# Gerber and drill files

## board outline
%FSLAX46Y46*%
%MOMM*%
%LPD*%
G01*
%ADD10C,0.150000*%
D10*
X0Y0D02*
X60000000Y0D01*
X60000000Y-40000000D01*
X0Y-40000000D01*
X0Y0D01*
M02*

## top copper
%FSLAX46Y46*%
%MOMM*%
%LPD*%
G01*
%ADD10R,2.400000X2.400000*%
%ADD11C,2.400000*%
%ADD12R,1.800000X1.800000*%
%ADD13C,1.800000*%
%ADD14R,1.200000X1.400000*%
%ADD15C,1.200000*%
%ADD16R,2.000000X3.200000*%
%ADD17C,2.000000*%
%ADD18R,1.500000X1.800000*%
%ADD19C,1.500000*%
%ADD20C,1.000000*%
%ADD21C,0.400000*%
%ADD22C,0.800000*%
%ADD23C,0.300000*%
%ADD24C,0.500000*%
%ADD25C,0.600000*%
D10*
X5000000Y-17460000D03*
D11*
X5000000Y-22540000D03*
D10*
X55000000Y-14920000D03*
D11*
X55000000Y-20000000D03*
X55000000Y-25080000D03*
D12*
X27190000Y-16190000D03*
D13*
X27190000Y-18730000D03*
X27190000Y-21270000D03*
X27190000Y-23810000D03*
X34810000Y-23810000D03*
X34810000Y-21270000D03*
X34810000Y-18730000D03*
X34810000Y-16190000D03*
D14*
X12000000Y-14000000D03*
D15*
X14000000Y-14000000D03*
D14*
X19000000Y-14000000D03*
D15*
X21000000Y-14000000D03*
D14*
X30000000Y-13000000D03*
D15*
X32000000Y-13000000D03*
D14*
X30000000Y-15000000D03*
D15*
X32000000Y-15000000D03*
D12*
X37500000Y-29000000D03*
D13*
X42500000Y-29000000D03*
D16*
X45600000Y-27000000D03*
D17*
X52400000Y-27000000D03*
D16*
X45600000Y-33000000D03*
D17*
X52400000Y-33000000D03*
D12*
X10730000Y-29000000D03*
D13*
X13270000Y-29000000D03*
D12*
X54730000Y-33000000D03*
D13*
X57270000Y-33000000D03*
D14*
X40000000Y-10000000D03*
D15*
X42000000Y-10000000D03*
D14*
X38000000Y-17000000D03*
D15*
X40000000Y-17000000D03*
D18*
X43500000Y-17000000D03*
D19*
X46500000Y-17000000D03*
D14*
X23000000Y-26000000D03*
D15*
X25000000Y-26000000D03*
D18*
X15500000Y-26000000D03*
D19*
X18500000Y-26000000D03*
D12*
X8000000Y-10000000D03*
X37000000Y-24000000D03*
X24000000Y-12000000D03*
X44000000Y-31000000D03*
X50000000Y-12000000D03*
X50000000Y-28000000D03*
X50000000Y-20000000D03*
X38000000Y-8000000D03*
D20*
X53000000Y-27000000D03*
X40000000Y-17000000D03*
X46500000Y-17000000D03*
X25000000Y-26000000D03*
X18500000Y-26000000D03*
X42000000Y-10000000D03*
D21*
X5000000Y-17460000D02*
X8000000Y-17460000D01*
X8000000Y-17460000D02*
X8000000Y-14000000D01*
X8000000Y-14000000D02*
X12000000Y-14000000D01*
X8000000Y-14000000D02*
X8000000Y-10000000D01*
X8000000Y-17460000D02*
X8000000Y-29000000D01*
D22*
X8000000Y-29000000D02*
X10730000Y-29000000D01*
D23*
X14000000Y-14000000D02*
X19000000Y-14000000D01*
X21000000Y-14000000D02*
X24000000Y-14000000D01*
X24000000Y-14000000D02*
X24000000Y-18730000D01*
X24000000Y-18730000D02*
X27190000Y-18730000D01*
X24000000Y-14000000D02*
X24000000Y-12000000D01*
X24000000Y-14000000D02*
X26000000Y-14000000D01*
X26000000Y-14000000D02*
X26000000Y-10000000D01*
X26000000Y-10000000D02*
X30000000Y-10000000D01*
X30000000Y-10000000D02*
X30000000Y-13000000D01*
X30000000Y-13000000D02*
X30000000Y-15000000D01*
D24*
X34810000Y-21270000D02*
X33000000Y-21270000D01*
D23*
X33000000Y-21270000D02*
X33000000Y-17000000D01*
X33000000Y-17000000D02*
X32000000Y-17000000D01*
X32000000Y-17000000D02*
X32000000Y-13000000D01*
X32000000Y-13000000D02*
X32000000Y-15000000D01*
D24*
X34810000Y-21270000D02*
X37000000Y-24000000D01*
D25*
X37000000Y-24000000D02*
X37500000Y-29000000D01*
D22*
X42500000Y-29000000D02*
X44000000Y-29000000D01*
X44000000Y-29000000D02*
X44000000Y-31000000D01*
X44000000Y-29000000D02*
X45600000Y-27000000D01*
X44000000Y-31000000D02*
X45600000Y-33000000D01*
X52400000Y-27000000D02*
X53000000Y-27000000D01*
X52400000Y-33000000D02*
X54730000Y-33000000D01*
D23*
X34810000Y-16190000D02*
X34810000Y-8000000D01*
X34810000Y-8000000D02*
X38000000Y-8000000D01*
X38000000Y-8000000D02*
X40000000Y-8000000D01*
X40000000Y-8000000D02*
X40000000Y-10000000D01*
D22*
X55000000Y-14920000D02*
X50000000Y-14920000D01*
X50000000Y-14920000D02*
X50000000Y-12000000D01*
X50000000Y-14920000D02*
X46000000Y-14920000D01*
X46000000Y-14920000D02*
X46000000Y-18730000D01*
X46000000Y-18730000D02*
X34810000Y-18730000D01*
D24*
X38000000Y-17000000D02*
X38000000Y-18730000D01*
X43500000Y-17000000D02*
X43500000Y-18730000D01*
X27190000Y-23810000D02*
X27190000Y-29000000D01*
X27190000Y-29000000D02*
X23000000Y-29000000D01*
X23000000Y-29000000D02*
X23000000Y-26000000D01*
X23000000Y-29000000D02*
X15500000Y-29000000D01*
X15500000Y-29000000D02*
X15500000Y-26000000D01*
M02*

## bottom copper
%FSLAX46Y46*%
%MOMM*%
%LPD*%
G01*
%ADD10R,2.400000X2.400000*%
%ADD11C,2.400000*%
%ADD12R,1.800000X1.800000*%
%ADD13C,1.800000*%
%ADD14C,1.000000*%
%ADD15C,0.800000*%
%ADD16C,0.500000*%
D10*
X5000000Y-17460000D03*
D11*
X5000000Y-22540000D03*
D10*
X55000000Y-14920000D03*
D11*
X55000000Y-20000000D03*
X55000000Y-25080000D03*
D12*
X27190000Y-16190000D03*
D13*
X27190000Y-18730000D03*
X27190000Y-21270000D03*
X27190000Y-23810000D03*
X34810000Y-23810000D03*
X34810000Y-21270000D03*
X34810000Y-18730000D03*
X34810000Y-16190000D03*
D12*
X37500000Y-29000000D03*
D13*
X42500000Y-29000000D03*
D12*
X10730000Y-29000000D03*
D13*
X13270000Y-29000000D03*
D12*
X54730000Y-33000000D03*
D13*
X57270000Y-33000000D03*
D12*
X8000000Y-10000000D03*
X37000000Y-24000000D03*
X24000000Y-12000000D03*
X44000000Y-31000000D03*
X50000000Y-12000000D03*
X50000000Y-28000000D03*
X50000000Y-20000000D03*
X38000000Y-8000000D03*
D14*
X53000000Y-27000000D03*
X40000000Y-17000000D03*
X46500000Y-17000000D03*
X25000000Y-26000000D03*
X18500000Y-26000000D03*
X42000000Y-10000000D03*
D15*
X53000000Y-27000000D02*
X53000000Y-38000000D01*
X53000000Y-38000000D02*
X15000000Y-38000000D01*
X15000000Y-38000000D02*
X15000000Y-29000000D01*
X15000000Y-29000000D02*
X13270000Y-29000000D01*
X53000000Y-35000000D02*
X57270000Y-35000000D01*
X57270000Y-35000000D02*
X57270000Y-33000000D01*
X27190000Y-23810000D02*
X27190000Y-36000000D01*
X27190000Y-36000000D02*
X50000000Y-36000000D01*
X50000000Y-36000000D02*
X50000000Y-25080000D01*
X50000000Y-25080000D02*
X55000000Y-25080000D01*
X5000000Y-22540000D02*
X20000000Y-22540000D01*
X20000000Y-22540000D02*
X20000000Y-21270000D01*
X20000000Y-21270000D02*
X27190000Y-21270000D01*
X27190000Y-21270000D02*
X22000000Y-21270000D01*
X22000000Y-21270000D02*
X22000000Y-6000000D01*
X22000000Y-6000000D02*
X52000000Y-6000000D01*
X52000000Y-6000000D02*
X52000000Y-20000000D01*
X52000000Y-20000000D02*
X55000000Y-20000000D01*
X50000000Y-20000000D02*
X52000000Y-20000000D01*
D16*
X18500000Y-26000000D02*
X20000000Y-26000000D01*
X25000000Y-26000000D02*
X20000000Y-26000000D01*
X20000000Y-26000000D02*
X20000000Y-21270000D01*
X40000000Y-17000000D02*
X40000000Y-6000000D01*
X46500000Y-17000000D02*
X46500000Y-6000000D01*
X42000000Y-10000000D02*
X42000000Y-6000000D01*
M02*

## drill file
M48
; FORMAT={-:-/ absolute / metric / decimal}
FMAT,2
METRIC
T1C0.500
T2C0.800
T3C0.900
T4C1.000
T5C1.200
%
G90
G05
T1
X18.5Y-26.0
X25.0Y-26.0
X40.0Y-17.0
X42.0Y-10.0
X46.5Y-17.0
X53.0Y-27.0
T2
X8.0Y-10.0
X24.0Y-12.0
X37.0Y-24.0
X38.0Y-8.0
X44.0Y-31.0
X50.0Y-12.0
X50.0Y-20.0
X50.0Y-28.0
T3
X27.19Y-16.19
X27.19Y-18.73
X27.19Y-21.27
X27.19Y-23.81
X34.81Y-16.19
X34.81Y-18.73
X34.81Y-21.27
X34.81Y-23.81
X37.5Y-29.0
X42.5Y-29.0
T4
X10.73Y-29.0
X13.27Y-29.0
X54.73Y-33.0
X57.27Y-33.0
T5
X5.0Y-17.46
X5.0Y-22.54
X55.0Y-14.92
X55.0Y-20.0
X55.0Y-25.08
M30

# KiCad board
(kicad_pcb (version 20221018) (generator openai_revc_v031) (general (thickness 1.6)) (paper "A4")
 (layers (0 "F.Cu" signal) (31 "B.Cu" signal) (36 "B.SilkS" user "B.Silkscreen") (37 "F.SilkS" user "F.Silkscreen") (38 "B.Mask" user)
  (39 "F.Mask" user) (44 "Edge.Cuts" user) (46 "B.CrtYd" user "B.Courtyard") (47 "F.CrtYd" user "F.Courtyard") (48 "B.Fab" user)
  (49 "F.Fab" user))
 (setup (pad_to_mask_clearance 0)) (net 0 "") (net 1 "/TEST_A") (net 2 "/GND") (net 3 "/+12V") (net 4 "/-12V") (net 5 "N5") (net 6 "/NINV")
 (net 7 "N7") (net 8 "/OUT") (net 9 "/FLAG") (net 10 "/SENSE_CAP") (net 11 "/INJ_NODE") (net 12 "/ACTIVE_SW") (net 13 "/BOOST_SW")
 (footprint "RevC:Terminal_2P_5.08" (layer "F.Cu") (at 5.00 20.00)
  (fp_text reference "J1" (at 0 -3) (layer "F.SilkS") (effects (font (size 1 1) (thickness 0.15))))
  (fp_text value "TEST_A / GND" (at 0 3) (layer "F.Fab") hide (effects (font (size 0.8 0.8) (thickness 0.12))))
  (pad "1" thru_hole rect (at 0.00 -2.54) (size 2.40 2.40) (drill 1.20) (layers "*.Cu" "*.Mask") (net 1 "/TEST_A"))
  (pad "2" thru_hole circle (at 0.00 2.54) (size 2.40 2.40) (drill 1.20) (layers "*.Cu" "*.Mask") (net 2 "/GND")))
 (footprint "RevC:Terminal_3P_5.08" (layer "F.Cu") (at 55.00 20.00)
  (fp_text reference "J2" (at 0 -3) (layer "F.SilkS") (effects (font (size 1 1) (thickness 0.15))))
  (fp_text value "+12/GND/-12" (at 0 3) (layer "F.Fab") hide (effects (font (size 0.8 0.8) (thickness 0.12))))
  (pad "1" thru_hole rect (at 0.00 -5.08) (size 2.40 2.40) (drill 1.20) (layers "*.Cu" "*.Mask") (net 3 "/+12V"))
  (pad "2" thru_hole circle (at 0.00 0.00) (size 2.40 2.40) (drill 1.20) (layers "*.Cu" "*.Mask") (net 2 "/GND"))
  (pad "3" thru_hole circle (at 0.00 5.08) (size 2.40 2.40) (drill 1.20) (layers "*.Cu" "*.Mask") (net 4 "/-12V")))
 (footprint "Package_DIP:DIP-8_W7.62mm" (layer "F.Cu") (at 31.00 20.00)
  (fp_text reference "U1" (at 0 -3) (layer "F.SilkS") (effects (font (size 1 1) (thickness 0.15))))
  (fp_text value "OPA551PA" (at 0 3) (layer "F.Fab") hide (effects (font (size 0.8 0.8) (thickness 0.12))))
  (pad "1" thru_hole rect (at -3.81 -3.81) (size 1.80 1.80) (drill 0.90) (layers "*.Cu" "*.Mask") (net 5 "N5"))
  (pad "2" thru_hole circle (at -3.81 -1.27) (size 1.80 1.80) (drill 0.90) (layers "*.Cu" "*.Mask") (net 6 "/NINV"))
  (pad "3" thru_hole circle (at -3.81 1.27) (size 1.80 1.80) (drill 0.90) (layers "*.Cu" "*.Mask") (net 2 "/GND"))
  (pad "4" thru_hole circle (at -3.81 3.81) (size 1.80 1.80) (drill 0.90) (layers "*.Cu" "*.Mask") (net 4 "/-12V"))
  (pad "5" thru_hole circle (at 3.81 3.81) (size 1.80 1.80) (drill 0.90) (layers "*.Cu" "*.Mask") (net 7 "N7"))
  (pad "6" thru_hole circle (at 3.81 1.27) (size 1.80 1.80) (drill 0.90) (layers "*.Cu" "*.Mask") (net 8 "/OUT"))
  (pad "7" thru_hole circle (at 3.81 -1.27) (size 1.80 1.80) (drill 0.90) (layers "*.Cu" "*.Mask") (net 3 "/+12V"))
  (pad "8" thru_hole circle (at 3.81 -3.81) (size 1.80 1.80) (drill 0.90) (layers "*.Cu" "*.Mask") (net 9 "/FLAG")))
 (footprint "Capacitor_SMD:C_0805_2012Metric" (layer "F.Cu") (at 13.00 14.00)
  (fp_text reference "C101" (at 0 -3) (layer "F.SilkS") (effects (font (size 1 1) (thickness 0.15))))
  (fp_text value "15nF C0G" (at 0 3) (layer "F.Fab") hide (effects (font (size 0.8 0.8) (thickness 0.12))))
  (pad "1" smd rect (at -1.00 0.00) (size 1.20 1.40) (layers "F.Cu" "F.Paste" "F.Mask") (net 1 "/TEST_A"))
  (pad "2" smd circle (at 1.00 0.00) (size 1.20 1.40) (layers "F.Cu" "F.Paste" "F.Mask") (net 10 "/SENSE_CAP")))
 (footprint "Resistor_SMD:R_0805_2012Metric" (layer "F.Cu") (at 20.00 14.00)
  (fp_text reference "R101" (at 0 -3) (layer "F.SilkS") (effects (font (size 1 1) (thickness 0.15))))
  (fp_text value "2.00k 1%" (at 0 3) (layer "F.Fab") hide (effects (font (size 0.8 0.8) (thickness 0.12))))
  (pad "1" smd rect (at -1.00 0.00) (size 1.20 1.40) (layers "F.Cu" "F.Paste" "F.Mask") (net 10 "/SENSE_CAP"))
  (pad "2" smd circle (at 1.00 0.00) (size 1.20 1.40) (layers "F.Cu" "F.Paste" "F.Mask") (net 6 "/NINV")))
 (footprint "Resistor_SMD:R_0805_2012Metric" (layer "F.Cu") (at 31.00 13.00)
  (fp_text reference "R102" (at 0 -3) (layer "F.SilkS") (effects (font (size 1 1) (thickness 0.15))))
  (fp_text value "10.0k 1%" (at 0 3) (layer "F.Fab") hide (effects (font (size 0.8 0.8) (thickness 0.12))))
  (pad "1" smd rect (at -1.00 0.00) (size 1.20 1.40) (layers "F.Cu" "F.Paste" "F.Mask") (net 6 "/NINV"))
  (pad "2" smd circle (at 1.00 0.00) (size 1.20 1.40) (layers "F.Cu" "F.Paste" "F.Mask") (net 8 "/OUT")))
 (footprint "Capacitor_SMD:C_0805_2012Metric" (layer "F.Cu") (at 31.00 15.00)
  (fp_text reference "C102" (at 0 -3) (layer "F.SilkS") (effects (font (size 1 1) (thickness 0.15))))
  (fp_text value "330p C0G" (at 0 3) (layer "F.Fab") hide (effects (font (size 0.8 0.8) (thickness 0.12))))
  (pad "1" smd rect (at -1.00 0.00) (size 1.20 1.40) (layers "F.Cu" "F.Paste" "F.Mask") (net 6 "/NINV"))
  (pad "2" smd circle (at 1.00 0.00) (size 1.20 1.40) (layers "F.Cu" "F.Paste" "F.Mask") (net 8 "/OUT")))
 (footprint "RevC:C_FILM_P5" (layer "F.Cu") (at 40.00 29.00)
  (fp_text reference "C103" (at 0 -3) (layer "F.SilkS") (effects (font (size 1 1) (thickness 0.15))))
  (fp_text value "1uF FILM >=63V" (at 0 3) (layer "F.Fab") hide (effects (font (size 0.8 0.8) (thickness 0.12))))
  (pad "1" thru_hole rect (at -2.50 0.00) (size 1.80 1.80) (drill 0.90) (layers "*.Cu" "*.Mask") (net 8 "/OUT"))
  (pad "2" thru_hole circle (at 2.50 0.00) (size 1.80 1.80) (drill 0.90) (layers "*.Cu" "*.Mask") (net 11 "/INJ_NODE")))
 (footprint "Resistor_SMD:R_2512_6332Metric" (layer "F.Cu") (at 49.00 27.00)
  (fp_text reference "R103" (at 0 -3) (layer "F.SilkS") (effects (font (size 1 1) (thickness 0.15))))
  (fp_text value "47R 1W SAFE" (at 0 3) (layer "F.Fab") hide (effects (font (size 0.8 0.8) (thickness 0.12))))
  (pad "1" smd rect (at -3.40 0.00) (size 2.00 3.20) (layers "F.Cu" "F.Paste" "F.Mask") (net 11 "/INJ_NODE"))
  (pad "2" smd circle (at 3.40 0.00) (size 2.00 3.20) (layers "F.Cu" "F.Paste" "F.Mask") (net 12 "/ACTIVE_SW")))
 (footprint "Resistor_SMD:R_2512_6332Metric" (layer "F.Cu") (at 49.00 33.00)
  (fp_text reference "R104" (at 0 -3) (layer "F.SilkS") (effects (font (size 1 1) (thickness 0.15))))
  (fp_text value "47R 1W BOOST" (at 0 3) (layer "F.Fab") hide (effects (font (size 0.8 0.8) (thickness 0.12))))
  (pad "1" smd rect (at -3.40 0.00) (size 2.00 3.20) (layers "F.Cu" "F.Paste" "F.Mask") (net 11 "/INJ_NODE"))
  (pad "2" smd circle (at 3.40 0.00) (size 2.00 3.20) (layers "F.Cu" "F.Paste" "F.Mask") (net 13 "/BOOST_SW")))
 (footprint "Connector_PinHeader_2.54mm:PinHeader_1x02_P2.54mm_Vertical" (layer "F.Cu") (at 12.00 29.00)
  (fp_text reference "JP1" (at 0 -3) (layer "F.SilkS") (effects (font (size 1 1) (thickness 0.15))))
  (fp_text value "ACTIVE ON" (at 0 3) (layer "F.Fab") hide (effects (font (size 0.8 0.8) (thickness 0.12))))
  (pad "1" thru_hole rect (at -1.27 0.00) (size 1.80 1.80) (drill 1.00) (layers "*.Cu" "*.Mask") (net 1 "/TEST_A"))
  (pad "2" thru_hole circle (at 1.27 0.00) (size 1.80 1.80) (drill 1.00) (layers "*.Cu" "*.Mask") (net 12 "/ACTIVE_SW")))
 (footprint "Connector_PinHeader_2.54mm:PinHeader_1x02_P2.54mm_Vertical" (layer "F.Cu") (at 56.00 33.00)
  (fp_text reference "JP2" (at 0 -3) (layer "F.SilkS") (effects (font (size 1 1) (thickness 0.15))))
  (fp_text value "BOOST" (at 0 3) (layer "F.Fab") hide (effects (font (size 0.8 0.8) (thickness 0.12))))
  (pad "1" thru_hole rect (at -1.27 0.00) (size 1.80 1.80) (drill 1.00) (layers "*.Cu" "*.Mask") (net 13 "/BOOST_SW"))
  (pad "2" thru_hole circle (at 1.27 0.00) (size 1.80 1.80) (drill 1.00) (layers "*.Cu" "*.Mask") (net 12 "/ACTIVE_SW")))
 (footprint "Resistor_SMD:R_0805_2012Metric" (layer "F.Cu") (at 41.00 10.00)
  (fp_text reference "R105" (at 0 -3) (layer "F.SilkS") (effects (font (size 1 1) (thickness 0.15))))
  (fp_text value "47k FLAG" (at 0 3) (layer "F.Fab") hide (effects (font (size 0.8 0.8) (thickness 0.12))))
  (pad "1" smd rect (at -1.00 0.00) (size 1.20 1.40) (layers "F.Cu" "F.Paste" "F.Mask") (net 9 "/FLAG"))
  (pad "2" smd circle (at 1.00 0.00) (size 1.20 1.40) (layers "F.Cu" "F.Paste" "F.Mask") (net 2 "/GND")))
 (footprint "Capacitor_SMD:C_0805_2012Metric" (layer "F.Cu") (at 39.00 17.00)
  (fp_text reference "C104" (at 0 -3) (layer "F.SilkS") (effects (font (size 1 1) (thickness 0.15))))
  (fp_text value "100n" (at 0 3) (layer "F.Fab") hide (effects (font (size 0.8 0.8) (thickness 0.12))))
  (pad "1" smd rect (at -1.00 0.00) (size 1.20 1.40) (layers "F.Cu" "F.Paste" "F.Mask") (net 3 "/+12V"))
  (pad "2" smd circle (at 1.00 0.00) (size 1.20 1.40) (layers "F.Cu" "F.Paste" "F.Mask") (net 2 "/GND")))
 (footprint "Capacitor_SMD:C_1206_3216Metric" (layer "F.Cu") (at 45.00 17.00)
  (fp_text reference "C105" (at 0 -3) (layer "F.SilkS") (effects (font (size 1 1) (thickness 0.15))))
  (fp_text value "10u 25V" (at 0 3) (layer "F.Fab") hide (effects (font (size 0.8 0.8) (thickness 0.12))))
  (pad "1" smd rect (at -1.50 0.00) (size 1.50 1.80) (layers "F.Cu" "F.Paste" "F.Mask") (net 3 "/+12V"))
  (pad "2" smd circle (at 1.50 0.00) (size 1.50 1.80) (layers "F.Cu" "F.Paste" "F.Mask") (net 2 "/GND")))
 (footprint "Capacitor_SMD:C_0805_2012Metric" (layer "F.Cu") (at 24.00 26.00)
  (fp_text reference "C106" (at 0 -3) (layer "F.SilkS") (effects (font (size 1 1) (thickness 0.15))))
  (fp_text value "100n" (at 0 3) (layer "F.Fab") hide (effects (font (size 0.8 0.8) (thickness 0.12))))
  (pad "1" smd rect (at -1.00 0.00) (size 1.20 1.40) (layers "F.Cu" "F.Paste" "F.Mask") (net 4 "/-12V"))
  (pad "2" smd circle (at 1.00 0.00) (size 1.20 1.40) (layers "F.Cu" "F.Paste" "F.Mask") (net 2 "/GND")))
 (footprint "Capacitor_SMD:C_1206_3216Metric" (layer "F.Cu") (at 17.00 26.00)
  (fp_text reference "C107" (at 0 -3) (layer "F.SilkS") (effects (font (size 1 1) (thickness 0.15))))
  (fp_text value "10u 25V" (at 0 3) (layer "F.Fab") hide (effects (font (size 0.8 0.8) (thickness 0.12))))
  (pad "1" smd rect (at -1.50 0.00) (size 1.50 1.80) (layers "F.Cu" "F.Paste" "F.Mask") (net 4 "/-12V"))
  (pad "2" smd circle (at 1.50 0.00) (size 1.50 1.80) (layers "F.Cu" "F.Paste" "F.Mask") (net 2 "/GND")))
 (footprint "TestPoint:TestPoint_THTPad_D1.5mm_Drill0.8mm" (layer "F.Cu") (at 8.00 10.00)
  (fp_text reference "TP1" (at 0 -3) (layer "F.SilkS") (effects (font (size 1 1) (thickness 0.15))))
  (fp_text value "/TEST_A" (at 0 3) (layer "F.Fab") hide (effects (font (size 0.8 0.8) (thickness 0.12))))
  (pad "1" thru_hole rect (at 0.00 0.00) (size 1.80 1.80) (drill 0.80) (layers "*.Cu" "*.Mask") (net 1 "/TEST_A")))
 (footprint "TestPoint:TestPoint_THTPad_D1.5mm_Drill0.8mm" (layer "F.Cu") (at 37.00 24.00)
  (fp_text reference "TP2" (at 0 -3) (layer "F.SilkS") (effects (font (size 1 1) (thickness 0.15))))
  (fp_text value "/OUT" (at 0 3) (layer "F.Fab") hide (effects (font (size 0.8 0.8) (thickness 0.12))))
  (pad "1" thru_hole rect (at 0.00 0.00) (size 1.80 1.80) (drill 0.80) (layers "*.Cu" "*.Mask") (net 8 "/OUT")))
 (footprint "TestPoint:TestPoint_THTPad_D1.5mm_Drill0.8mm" (layer "F.Cu") (at 24.00 12.00)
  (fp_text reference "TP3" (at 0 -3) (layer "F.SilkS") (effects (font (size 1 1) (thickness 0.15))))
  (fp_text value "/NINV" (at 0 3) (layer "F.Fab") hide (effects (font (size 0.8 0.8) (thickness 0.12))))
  (pad "1" thru_hole rect (at 0.00 0.00) (size 1.80 1.80) (drill 0.80) (layers "*.Cu" "*.Mask") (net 6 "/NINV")))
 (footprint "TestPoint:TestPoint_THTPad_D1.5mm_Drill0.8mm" (layer "F.Cu") (at 44.00 31.00)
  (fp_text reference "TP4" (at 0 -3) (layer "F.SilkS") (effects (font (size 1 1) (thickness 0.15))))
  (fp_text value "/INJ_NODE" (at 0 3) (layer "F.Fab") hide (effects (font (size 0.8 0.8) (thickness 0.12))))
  (pad "1" thru_hole rect (at 0.00 0.00) (size 1.80 1.80) (drill 0.80) (layers "*.Cu" "*.Mask") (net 11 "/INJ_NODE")))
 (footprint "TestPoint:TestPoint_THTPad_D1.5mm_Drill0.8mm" (layer "F.Cu") (at 50.00 12.00)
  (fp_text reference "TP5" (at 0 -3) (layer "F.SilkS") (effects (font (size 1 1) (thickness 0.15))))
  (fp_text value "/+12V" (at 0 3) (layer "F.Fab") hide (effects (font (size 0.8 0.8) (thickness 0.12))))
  (pad "1" thru_hole rect (at 0.00 0.00) (size 1.80 1.80) (drill 0.80) (layers "*.Cu" "*.Mask") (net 3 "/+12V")))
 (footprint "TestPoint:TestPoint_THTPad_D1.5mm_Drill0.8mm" (layer "F.Cu") (at 50.00 28.00)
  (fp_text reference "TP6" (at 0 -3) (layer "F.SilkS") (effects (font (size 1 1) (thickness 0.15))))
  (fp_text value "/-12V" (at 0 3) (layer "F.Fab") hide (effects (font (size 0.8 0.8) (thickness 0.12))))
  (pad "1" thru_hole rect (at 0.00 0.00) (size 1.80 1.80) (drill 0.80) (layers "*.Cu" "*.Mask") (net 4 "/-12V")))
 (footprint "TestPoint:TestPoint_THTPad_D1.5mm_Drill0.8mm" (layer "F.Cu") (at 50.00 20.00)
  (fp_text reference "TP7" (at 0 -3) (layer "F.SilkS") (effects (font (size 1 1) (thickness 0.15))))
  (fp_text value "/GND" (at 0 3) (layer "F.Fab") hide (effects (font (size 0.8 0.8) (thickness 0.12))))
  (pad "1" thru_hole rect (at 0.00 0.00) (size 1.80 1.80) (drill 0.80) (layers "*.Cu" "*.Mask") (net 2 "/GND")))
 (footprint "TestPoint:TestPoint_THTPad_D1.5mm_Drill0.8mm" (layer "F.Cu") (at 38.00 8.00)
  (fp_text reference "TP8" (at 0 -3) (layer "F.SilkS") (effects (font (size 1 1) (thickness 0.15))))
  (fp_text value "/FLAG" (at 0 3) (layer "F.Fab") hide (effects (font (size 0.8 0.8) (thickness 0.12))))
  (pad "1" thru_hole rect (at 0.00 0.00) (size 1.80 1.80) (drill 0.80) (layers "*.Cu" "*.Mask") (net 9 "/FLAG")))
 (gr_rect (start 0 0) (end 60 40) (stroke (width 0.15) (type default)) (fill none) (layer "Edge.Cuts"))
 (segment (start 5.00 17.46) (end 8.00 17.46) (width 0.40) (layer "F.Cu") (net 1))
 (segment (start 8.00 17.46) (end 8.00 14.00) (width 0.40) (layer "F.Cu") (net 1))
 (segment (start 8.00 14.00) (end 12.00 14.00) (width 0.40) (layer "F.Cu") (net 1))
 (segment (start 8.00 14.00) (end 8.00 10.00) (width 0.40) (layer "F.Cu") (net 1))
 (segment (start 8.00 17.46) (end 8.00 29.00) (width 0.40) (layer "F.Cu") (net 1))
 (segment (start 8.00 29.00) (end 10.73 29.00) (width 0.80) (layer "F.Cu") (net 1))
 (segment (start 14.00 14.00) (end 19.00 14.00) (width 0.30) (layer "F.Cu") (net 10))
 (segment (start 21.00 14.00) (end 24.00 14.00) (width 0.30) (layer "F.Cu") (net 6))
 (segment (start 24.00 14.00) (end 24.00 18.73) (width 0.30) (layer "F.Cu") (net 6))
 (segment (start 24.00 18.73) (end 27.19 18.73) (width 0.30) (layer "F.Cu") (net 6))
 (segment (start 24.00 14.00) (end 24.00 12.00) (width 0.30) (layer "F.Cu") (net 6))
 (segment (start 24.00 14.00) (end 26.00 14.00) (width 0.30) (layer "F.Cu") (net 6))
 (segment (start 26.00 14.00) (end 26.00 10.00) (width 0.30) (layer "F.Cu") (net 6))
 (segment (start 26.00 10.00) (end 30.00 10.00) (width 0.30) (layer "F.Cu") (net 6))
 (segment (start 30.00 10.00) (end 30.00 13.00) (width 0.30) (layer "F.Cu") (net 6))
 (segment (start 30.00 13.00) (end 30.00 15.00) (width 0.30) (layer "F.Cu") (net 6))
 (segment (start 34.81 21.27) (end 33.00 21.27) (width 0.50) (layer "F.Cu") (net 8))
 (segment (start 33.00 21.27) (end 33.00 17.00) (width 0.30) (layer "F.Cu") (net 8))
 (segment (start 33.00 17.00) (end 32.00 17.00) (width 0.30) (layer "F.Cu") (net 8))
 (segment (start 32.00 17.00) (end 32.00 13.00) (width 0.30) (layer "F.Cu") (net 8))
 (segment (start 32.00 13.00) (end 32.00 15.00) (width 0.30) (layer "F.Cu") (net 8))
 (segment (start 34.81 21.27) (end 37.00 24.00) (width 0.50) (layer "F.Cu") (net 8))
 (segment (start 37.00 24.00) (end 37.50 29.00) (width 0.60) (layer "F.Cu") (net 8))
 (segment (start 42.50 29.00) (end 44.00 29.00) (width 0.80) (layer "F.Cu") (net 11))
 (segment (start 44.00 29.00) (end 44.00 31.00) (width 0.80) (layer "F.Cu") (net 11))
 (segment (start 44.00 29.00) (end 45.60 27.00) (width 0.80) (layer "F.Cu") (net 11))
 (segment (start 44.00 31.00) (end 45.60 33.00) (width 0.80) (layer "F.Cu") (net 11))
 (segment (start 52.40 27.00) (end 53.00 27.00) (width 0.80) (layer "F.Cu") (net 12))
 (via (at 53.00 27.00) (size 1.0) (drill 0.5) (layers "F.Cu" "B.Cu") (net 12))
 (segment (start 53.00 27.00) (end 53.00 38.00) (width 0.80) (layer "B.Cu") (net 12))
 (segment (start 53.00 38.00) (end 15.00 38.00) (width 0.80) (layer "B.Cu") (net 12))
 (segment (start 15.00 38.00) (end 15.00 29.00) (width 0.80) (layer "B.Cu") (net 12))
 (segment (start 15.00 29.00) (end 13.27 29.00) (width 0.80) (layer "B.Cu") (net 12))
 (segment (start 53.00 35.00) (end 57.27 35.00) (width 0.80) (layer "B.Cu") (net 12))
 (segment (start 57.27 35.00) (end 57.27 33.00) (width 0.80) (layer "B.Cu") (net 12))
 (segment (start 52.40 33.00) (end 54.73 33.00) (width 0.80) (layer "F.Cu") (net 13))
 (segment (start 34.81 16.19) (end 34.81 8.00) (width 0.30) (layer "F.Cu") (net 9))
 (segment (start 34.81 8.00) (end 38.00 8.00) (width 0.30) (layer "F.Cu") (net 9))
 (segment (start 38.00 8.00) (end 40.00 8.00) (width 0.30) (layer "F.Cu") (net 9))
 (segment (start 40.00 8.00) (end 40.00 10.00) (width 0.30) (layer "F.Cu") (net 9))
 (segment (start 55.00 14.92) (end 50.00 14.92) (width 0.80) (layer "F.Cu") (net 3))
 (segment (start 50.00 14.92) (end 50.00 12.00) (width 0.80) (layer "F.Cu") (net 3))
 (segment (start 50.00 14.92) (end 46.00 14.92) (width 0.80) (layer "F.Cu") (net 3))
 (segment (start 46.00 14.92) (end 46.00 18.73) (width 0.80) (layer "F.Cu") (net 3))
 (segment (start 46.00 18.73) (end 34.81 18.73) (width 0.80) (layer "F.Cu") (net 3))
 (segment (start 38.00 17.00) (end 38.00 18.73) (width 0.50) (layer "F.Cu") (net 3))
 (segment (start 43.50 17.00) (end 43.50 18.73) (width 0.50) (layer "F.Cu") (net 3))
 (segment (start 27.19 23.81) (end 27.19 36.00) (width 0.80) (layer "B.Cu") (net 4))
 (segment (start 27.19 36.00) (end 50.00 36.00) (width 0.80) (layer "B.Cu") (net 4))
 (segment (start 50.00 36.00) (end 50.00 25.08) (width 0.80) (layer "B.Cu") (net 4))
 (segment (start 50.00 25.08) (end 55.00 25.08) (width 0.80) (layer "B.Cu") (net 4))
 (segment (start 27.19 23.81) (end 27.19 29.00) (width 0.50) (layer "F.Cu") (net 4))
 (segment (start 27.19 29.00) (end 23.00 29.00) (width 0.50) (layer "F.Cu") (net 4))
 (segment (start 23.00 29.00) (end 23.00 26.00) (width 0.50) (layer "F.Cu") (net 4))
 (segment (start 23.00 29.00) (end 15.50 29.00) (width 0.50) (layer "F.Cu") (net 4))
 (segment (start 15.50 29.00) (end 15.50 26.00) (width 0.50) (layer "F.Cu") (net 4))
 (via (at 40.00 17.00) (size 1.0) (drill 0.5) (layers "F.Cu" "B.Cu") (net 2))
 (via (at 46.50 17.00) (size 1.0) (drill 0.5) (layers "F.Cu" "B.Cu") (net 2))
 (via (at 25.00 26.00) (size 1.0) (drill 0.5) (layers "F.Cu" "B.Cu") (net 2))
 (via (at 18.50 26.00) (size 1.0) (drill 0.5) (layers "F.Cu" "B.Cu") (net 2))
 (via (at 42.00 10.00) (size 1.0) (drill 0.5) (layers "F.Cu" "B.Cu") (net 2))
 (segment (start 5.00 22.54) (end 20.00 22.54) (width 0.80) (layer "B.Cu") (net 2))
 (segment (start 20.00 22.54) (end 20.00 21.27) (width 0.80) (layer "B.Cu") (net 2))
 (segment (start 20.00 21.27) (end 27.19 21.27) (width 0.80) (layer "B.Cu") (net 2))
 (segment (start 27.19 21.27) (end 22.00 21.27) (width 0.80) (layer "B.Cu") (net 2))
 (segment (start 22.00 21.27) (end 22.00 6.00) (width 0.80) (layer "B.Cu") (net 2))
 (segment (start 22.00 6.00) (end 52.00 6.00) (width 0.80) (layer "B.Cu") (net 2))
 (segment (start 52.00 6.00) (end 52.00 20.00) (width 0.80) (layer "B.Cu") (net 2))
 (segment (start 52.00 20.00) (end 55.00 20.00) (width 0.80) (layer "B.Cu") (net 2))
 (segment (start 50.00 20.00) (end 52.00 20.00) (width 0.80) (layer "B.Cu") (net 2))
 (segment (start 18.50 26.00) (end 20.00 26.00) (width 0.50) (layer "B.Cu") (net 2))
 (segment (start 25.00 26.00) (end 20.00 26.00) (width 0.50) (layer "B.Cu") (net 2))
 (segment (start 20.00 26.00) (end 20.00 21.27) (width 0.50) (layer "B.Cu") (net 2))
 (segment (start 40.00 17.00) (end 40.00 6.00) (width 0.50) (layer "B.Cu") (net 2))
 (segment (start 46.50 17.00) (end 46.50 6.00) (width 0.50) (layer "B.Cu") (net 2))
 (segment (start 42.00 10.00) (end 42.00 6.00) (width 0.50) (layer "B.Cu") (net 2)))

